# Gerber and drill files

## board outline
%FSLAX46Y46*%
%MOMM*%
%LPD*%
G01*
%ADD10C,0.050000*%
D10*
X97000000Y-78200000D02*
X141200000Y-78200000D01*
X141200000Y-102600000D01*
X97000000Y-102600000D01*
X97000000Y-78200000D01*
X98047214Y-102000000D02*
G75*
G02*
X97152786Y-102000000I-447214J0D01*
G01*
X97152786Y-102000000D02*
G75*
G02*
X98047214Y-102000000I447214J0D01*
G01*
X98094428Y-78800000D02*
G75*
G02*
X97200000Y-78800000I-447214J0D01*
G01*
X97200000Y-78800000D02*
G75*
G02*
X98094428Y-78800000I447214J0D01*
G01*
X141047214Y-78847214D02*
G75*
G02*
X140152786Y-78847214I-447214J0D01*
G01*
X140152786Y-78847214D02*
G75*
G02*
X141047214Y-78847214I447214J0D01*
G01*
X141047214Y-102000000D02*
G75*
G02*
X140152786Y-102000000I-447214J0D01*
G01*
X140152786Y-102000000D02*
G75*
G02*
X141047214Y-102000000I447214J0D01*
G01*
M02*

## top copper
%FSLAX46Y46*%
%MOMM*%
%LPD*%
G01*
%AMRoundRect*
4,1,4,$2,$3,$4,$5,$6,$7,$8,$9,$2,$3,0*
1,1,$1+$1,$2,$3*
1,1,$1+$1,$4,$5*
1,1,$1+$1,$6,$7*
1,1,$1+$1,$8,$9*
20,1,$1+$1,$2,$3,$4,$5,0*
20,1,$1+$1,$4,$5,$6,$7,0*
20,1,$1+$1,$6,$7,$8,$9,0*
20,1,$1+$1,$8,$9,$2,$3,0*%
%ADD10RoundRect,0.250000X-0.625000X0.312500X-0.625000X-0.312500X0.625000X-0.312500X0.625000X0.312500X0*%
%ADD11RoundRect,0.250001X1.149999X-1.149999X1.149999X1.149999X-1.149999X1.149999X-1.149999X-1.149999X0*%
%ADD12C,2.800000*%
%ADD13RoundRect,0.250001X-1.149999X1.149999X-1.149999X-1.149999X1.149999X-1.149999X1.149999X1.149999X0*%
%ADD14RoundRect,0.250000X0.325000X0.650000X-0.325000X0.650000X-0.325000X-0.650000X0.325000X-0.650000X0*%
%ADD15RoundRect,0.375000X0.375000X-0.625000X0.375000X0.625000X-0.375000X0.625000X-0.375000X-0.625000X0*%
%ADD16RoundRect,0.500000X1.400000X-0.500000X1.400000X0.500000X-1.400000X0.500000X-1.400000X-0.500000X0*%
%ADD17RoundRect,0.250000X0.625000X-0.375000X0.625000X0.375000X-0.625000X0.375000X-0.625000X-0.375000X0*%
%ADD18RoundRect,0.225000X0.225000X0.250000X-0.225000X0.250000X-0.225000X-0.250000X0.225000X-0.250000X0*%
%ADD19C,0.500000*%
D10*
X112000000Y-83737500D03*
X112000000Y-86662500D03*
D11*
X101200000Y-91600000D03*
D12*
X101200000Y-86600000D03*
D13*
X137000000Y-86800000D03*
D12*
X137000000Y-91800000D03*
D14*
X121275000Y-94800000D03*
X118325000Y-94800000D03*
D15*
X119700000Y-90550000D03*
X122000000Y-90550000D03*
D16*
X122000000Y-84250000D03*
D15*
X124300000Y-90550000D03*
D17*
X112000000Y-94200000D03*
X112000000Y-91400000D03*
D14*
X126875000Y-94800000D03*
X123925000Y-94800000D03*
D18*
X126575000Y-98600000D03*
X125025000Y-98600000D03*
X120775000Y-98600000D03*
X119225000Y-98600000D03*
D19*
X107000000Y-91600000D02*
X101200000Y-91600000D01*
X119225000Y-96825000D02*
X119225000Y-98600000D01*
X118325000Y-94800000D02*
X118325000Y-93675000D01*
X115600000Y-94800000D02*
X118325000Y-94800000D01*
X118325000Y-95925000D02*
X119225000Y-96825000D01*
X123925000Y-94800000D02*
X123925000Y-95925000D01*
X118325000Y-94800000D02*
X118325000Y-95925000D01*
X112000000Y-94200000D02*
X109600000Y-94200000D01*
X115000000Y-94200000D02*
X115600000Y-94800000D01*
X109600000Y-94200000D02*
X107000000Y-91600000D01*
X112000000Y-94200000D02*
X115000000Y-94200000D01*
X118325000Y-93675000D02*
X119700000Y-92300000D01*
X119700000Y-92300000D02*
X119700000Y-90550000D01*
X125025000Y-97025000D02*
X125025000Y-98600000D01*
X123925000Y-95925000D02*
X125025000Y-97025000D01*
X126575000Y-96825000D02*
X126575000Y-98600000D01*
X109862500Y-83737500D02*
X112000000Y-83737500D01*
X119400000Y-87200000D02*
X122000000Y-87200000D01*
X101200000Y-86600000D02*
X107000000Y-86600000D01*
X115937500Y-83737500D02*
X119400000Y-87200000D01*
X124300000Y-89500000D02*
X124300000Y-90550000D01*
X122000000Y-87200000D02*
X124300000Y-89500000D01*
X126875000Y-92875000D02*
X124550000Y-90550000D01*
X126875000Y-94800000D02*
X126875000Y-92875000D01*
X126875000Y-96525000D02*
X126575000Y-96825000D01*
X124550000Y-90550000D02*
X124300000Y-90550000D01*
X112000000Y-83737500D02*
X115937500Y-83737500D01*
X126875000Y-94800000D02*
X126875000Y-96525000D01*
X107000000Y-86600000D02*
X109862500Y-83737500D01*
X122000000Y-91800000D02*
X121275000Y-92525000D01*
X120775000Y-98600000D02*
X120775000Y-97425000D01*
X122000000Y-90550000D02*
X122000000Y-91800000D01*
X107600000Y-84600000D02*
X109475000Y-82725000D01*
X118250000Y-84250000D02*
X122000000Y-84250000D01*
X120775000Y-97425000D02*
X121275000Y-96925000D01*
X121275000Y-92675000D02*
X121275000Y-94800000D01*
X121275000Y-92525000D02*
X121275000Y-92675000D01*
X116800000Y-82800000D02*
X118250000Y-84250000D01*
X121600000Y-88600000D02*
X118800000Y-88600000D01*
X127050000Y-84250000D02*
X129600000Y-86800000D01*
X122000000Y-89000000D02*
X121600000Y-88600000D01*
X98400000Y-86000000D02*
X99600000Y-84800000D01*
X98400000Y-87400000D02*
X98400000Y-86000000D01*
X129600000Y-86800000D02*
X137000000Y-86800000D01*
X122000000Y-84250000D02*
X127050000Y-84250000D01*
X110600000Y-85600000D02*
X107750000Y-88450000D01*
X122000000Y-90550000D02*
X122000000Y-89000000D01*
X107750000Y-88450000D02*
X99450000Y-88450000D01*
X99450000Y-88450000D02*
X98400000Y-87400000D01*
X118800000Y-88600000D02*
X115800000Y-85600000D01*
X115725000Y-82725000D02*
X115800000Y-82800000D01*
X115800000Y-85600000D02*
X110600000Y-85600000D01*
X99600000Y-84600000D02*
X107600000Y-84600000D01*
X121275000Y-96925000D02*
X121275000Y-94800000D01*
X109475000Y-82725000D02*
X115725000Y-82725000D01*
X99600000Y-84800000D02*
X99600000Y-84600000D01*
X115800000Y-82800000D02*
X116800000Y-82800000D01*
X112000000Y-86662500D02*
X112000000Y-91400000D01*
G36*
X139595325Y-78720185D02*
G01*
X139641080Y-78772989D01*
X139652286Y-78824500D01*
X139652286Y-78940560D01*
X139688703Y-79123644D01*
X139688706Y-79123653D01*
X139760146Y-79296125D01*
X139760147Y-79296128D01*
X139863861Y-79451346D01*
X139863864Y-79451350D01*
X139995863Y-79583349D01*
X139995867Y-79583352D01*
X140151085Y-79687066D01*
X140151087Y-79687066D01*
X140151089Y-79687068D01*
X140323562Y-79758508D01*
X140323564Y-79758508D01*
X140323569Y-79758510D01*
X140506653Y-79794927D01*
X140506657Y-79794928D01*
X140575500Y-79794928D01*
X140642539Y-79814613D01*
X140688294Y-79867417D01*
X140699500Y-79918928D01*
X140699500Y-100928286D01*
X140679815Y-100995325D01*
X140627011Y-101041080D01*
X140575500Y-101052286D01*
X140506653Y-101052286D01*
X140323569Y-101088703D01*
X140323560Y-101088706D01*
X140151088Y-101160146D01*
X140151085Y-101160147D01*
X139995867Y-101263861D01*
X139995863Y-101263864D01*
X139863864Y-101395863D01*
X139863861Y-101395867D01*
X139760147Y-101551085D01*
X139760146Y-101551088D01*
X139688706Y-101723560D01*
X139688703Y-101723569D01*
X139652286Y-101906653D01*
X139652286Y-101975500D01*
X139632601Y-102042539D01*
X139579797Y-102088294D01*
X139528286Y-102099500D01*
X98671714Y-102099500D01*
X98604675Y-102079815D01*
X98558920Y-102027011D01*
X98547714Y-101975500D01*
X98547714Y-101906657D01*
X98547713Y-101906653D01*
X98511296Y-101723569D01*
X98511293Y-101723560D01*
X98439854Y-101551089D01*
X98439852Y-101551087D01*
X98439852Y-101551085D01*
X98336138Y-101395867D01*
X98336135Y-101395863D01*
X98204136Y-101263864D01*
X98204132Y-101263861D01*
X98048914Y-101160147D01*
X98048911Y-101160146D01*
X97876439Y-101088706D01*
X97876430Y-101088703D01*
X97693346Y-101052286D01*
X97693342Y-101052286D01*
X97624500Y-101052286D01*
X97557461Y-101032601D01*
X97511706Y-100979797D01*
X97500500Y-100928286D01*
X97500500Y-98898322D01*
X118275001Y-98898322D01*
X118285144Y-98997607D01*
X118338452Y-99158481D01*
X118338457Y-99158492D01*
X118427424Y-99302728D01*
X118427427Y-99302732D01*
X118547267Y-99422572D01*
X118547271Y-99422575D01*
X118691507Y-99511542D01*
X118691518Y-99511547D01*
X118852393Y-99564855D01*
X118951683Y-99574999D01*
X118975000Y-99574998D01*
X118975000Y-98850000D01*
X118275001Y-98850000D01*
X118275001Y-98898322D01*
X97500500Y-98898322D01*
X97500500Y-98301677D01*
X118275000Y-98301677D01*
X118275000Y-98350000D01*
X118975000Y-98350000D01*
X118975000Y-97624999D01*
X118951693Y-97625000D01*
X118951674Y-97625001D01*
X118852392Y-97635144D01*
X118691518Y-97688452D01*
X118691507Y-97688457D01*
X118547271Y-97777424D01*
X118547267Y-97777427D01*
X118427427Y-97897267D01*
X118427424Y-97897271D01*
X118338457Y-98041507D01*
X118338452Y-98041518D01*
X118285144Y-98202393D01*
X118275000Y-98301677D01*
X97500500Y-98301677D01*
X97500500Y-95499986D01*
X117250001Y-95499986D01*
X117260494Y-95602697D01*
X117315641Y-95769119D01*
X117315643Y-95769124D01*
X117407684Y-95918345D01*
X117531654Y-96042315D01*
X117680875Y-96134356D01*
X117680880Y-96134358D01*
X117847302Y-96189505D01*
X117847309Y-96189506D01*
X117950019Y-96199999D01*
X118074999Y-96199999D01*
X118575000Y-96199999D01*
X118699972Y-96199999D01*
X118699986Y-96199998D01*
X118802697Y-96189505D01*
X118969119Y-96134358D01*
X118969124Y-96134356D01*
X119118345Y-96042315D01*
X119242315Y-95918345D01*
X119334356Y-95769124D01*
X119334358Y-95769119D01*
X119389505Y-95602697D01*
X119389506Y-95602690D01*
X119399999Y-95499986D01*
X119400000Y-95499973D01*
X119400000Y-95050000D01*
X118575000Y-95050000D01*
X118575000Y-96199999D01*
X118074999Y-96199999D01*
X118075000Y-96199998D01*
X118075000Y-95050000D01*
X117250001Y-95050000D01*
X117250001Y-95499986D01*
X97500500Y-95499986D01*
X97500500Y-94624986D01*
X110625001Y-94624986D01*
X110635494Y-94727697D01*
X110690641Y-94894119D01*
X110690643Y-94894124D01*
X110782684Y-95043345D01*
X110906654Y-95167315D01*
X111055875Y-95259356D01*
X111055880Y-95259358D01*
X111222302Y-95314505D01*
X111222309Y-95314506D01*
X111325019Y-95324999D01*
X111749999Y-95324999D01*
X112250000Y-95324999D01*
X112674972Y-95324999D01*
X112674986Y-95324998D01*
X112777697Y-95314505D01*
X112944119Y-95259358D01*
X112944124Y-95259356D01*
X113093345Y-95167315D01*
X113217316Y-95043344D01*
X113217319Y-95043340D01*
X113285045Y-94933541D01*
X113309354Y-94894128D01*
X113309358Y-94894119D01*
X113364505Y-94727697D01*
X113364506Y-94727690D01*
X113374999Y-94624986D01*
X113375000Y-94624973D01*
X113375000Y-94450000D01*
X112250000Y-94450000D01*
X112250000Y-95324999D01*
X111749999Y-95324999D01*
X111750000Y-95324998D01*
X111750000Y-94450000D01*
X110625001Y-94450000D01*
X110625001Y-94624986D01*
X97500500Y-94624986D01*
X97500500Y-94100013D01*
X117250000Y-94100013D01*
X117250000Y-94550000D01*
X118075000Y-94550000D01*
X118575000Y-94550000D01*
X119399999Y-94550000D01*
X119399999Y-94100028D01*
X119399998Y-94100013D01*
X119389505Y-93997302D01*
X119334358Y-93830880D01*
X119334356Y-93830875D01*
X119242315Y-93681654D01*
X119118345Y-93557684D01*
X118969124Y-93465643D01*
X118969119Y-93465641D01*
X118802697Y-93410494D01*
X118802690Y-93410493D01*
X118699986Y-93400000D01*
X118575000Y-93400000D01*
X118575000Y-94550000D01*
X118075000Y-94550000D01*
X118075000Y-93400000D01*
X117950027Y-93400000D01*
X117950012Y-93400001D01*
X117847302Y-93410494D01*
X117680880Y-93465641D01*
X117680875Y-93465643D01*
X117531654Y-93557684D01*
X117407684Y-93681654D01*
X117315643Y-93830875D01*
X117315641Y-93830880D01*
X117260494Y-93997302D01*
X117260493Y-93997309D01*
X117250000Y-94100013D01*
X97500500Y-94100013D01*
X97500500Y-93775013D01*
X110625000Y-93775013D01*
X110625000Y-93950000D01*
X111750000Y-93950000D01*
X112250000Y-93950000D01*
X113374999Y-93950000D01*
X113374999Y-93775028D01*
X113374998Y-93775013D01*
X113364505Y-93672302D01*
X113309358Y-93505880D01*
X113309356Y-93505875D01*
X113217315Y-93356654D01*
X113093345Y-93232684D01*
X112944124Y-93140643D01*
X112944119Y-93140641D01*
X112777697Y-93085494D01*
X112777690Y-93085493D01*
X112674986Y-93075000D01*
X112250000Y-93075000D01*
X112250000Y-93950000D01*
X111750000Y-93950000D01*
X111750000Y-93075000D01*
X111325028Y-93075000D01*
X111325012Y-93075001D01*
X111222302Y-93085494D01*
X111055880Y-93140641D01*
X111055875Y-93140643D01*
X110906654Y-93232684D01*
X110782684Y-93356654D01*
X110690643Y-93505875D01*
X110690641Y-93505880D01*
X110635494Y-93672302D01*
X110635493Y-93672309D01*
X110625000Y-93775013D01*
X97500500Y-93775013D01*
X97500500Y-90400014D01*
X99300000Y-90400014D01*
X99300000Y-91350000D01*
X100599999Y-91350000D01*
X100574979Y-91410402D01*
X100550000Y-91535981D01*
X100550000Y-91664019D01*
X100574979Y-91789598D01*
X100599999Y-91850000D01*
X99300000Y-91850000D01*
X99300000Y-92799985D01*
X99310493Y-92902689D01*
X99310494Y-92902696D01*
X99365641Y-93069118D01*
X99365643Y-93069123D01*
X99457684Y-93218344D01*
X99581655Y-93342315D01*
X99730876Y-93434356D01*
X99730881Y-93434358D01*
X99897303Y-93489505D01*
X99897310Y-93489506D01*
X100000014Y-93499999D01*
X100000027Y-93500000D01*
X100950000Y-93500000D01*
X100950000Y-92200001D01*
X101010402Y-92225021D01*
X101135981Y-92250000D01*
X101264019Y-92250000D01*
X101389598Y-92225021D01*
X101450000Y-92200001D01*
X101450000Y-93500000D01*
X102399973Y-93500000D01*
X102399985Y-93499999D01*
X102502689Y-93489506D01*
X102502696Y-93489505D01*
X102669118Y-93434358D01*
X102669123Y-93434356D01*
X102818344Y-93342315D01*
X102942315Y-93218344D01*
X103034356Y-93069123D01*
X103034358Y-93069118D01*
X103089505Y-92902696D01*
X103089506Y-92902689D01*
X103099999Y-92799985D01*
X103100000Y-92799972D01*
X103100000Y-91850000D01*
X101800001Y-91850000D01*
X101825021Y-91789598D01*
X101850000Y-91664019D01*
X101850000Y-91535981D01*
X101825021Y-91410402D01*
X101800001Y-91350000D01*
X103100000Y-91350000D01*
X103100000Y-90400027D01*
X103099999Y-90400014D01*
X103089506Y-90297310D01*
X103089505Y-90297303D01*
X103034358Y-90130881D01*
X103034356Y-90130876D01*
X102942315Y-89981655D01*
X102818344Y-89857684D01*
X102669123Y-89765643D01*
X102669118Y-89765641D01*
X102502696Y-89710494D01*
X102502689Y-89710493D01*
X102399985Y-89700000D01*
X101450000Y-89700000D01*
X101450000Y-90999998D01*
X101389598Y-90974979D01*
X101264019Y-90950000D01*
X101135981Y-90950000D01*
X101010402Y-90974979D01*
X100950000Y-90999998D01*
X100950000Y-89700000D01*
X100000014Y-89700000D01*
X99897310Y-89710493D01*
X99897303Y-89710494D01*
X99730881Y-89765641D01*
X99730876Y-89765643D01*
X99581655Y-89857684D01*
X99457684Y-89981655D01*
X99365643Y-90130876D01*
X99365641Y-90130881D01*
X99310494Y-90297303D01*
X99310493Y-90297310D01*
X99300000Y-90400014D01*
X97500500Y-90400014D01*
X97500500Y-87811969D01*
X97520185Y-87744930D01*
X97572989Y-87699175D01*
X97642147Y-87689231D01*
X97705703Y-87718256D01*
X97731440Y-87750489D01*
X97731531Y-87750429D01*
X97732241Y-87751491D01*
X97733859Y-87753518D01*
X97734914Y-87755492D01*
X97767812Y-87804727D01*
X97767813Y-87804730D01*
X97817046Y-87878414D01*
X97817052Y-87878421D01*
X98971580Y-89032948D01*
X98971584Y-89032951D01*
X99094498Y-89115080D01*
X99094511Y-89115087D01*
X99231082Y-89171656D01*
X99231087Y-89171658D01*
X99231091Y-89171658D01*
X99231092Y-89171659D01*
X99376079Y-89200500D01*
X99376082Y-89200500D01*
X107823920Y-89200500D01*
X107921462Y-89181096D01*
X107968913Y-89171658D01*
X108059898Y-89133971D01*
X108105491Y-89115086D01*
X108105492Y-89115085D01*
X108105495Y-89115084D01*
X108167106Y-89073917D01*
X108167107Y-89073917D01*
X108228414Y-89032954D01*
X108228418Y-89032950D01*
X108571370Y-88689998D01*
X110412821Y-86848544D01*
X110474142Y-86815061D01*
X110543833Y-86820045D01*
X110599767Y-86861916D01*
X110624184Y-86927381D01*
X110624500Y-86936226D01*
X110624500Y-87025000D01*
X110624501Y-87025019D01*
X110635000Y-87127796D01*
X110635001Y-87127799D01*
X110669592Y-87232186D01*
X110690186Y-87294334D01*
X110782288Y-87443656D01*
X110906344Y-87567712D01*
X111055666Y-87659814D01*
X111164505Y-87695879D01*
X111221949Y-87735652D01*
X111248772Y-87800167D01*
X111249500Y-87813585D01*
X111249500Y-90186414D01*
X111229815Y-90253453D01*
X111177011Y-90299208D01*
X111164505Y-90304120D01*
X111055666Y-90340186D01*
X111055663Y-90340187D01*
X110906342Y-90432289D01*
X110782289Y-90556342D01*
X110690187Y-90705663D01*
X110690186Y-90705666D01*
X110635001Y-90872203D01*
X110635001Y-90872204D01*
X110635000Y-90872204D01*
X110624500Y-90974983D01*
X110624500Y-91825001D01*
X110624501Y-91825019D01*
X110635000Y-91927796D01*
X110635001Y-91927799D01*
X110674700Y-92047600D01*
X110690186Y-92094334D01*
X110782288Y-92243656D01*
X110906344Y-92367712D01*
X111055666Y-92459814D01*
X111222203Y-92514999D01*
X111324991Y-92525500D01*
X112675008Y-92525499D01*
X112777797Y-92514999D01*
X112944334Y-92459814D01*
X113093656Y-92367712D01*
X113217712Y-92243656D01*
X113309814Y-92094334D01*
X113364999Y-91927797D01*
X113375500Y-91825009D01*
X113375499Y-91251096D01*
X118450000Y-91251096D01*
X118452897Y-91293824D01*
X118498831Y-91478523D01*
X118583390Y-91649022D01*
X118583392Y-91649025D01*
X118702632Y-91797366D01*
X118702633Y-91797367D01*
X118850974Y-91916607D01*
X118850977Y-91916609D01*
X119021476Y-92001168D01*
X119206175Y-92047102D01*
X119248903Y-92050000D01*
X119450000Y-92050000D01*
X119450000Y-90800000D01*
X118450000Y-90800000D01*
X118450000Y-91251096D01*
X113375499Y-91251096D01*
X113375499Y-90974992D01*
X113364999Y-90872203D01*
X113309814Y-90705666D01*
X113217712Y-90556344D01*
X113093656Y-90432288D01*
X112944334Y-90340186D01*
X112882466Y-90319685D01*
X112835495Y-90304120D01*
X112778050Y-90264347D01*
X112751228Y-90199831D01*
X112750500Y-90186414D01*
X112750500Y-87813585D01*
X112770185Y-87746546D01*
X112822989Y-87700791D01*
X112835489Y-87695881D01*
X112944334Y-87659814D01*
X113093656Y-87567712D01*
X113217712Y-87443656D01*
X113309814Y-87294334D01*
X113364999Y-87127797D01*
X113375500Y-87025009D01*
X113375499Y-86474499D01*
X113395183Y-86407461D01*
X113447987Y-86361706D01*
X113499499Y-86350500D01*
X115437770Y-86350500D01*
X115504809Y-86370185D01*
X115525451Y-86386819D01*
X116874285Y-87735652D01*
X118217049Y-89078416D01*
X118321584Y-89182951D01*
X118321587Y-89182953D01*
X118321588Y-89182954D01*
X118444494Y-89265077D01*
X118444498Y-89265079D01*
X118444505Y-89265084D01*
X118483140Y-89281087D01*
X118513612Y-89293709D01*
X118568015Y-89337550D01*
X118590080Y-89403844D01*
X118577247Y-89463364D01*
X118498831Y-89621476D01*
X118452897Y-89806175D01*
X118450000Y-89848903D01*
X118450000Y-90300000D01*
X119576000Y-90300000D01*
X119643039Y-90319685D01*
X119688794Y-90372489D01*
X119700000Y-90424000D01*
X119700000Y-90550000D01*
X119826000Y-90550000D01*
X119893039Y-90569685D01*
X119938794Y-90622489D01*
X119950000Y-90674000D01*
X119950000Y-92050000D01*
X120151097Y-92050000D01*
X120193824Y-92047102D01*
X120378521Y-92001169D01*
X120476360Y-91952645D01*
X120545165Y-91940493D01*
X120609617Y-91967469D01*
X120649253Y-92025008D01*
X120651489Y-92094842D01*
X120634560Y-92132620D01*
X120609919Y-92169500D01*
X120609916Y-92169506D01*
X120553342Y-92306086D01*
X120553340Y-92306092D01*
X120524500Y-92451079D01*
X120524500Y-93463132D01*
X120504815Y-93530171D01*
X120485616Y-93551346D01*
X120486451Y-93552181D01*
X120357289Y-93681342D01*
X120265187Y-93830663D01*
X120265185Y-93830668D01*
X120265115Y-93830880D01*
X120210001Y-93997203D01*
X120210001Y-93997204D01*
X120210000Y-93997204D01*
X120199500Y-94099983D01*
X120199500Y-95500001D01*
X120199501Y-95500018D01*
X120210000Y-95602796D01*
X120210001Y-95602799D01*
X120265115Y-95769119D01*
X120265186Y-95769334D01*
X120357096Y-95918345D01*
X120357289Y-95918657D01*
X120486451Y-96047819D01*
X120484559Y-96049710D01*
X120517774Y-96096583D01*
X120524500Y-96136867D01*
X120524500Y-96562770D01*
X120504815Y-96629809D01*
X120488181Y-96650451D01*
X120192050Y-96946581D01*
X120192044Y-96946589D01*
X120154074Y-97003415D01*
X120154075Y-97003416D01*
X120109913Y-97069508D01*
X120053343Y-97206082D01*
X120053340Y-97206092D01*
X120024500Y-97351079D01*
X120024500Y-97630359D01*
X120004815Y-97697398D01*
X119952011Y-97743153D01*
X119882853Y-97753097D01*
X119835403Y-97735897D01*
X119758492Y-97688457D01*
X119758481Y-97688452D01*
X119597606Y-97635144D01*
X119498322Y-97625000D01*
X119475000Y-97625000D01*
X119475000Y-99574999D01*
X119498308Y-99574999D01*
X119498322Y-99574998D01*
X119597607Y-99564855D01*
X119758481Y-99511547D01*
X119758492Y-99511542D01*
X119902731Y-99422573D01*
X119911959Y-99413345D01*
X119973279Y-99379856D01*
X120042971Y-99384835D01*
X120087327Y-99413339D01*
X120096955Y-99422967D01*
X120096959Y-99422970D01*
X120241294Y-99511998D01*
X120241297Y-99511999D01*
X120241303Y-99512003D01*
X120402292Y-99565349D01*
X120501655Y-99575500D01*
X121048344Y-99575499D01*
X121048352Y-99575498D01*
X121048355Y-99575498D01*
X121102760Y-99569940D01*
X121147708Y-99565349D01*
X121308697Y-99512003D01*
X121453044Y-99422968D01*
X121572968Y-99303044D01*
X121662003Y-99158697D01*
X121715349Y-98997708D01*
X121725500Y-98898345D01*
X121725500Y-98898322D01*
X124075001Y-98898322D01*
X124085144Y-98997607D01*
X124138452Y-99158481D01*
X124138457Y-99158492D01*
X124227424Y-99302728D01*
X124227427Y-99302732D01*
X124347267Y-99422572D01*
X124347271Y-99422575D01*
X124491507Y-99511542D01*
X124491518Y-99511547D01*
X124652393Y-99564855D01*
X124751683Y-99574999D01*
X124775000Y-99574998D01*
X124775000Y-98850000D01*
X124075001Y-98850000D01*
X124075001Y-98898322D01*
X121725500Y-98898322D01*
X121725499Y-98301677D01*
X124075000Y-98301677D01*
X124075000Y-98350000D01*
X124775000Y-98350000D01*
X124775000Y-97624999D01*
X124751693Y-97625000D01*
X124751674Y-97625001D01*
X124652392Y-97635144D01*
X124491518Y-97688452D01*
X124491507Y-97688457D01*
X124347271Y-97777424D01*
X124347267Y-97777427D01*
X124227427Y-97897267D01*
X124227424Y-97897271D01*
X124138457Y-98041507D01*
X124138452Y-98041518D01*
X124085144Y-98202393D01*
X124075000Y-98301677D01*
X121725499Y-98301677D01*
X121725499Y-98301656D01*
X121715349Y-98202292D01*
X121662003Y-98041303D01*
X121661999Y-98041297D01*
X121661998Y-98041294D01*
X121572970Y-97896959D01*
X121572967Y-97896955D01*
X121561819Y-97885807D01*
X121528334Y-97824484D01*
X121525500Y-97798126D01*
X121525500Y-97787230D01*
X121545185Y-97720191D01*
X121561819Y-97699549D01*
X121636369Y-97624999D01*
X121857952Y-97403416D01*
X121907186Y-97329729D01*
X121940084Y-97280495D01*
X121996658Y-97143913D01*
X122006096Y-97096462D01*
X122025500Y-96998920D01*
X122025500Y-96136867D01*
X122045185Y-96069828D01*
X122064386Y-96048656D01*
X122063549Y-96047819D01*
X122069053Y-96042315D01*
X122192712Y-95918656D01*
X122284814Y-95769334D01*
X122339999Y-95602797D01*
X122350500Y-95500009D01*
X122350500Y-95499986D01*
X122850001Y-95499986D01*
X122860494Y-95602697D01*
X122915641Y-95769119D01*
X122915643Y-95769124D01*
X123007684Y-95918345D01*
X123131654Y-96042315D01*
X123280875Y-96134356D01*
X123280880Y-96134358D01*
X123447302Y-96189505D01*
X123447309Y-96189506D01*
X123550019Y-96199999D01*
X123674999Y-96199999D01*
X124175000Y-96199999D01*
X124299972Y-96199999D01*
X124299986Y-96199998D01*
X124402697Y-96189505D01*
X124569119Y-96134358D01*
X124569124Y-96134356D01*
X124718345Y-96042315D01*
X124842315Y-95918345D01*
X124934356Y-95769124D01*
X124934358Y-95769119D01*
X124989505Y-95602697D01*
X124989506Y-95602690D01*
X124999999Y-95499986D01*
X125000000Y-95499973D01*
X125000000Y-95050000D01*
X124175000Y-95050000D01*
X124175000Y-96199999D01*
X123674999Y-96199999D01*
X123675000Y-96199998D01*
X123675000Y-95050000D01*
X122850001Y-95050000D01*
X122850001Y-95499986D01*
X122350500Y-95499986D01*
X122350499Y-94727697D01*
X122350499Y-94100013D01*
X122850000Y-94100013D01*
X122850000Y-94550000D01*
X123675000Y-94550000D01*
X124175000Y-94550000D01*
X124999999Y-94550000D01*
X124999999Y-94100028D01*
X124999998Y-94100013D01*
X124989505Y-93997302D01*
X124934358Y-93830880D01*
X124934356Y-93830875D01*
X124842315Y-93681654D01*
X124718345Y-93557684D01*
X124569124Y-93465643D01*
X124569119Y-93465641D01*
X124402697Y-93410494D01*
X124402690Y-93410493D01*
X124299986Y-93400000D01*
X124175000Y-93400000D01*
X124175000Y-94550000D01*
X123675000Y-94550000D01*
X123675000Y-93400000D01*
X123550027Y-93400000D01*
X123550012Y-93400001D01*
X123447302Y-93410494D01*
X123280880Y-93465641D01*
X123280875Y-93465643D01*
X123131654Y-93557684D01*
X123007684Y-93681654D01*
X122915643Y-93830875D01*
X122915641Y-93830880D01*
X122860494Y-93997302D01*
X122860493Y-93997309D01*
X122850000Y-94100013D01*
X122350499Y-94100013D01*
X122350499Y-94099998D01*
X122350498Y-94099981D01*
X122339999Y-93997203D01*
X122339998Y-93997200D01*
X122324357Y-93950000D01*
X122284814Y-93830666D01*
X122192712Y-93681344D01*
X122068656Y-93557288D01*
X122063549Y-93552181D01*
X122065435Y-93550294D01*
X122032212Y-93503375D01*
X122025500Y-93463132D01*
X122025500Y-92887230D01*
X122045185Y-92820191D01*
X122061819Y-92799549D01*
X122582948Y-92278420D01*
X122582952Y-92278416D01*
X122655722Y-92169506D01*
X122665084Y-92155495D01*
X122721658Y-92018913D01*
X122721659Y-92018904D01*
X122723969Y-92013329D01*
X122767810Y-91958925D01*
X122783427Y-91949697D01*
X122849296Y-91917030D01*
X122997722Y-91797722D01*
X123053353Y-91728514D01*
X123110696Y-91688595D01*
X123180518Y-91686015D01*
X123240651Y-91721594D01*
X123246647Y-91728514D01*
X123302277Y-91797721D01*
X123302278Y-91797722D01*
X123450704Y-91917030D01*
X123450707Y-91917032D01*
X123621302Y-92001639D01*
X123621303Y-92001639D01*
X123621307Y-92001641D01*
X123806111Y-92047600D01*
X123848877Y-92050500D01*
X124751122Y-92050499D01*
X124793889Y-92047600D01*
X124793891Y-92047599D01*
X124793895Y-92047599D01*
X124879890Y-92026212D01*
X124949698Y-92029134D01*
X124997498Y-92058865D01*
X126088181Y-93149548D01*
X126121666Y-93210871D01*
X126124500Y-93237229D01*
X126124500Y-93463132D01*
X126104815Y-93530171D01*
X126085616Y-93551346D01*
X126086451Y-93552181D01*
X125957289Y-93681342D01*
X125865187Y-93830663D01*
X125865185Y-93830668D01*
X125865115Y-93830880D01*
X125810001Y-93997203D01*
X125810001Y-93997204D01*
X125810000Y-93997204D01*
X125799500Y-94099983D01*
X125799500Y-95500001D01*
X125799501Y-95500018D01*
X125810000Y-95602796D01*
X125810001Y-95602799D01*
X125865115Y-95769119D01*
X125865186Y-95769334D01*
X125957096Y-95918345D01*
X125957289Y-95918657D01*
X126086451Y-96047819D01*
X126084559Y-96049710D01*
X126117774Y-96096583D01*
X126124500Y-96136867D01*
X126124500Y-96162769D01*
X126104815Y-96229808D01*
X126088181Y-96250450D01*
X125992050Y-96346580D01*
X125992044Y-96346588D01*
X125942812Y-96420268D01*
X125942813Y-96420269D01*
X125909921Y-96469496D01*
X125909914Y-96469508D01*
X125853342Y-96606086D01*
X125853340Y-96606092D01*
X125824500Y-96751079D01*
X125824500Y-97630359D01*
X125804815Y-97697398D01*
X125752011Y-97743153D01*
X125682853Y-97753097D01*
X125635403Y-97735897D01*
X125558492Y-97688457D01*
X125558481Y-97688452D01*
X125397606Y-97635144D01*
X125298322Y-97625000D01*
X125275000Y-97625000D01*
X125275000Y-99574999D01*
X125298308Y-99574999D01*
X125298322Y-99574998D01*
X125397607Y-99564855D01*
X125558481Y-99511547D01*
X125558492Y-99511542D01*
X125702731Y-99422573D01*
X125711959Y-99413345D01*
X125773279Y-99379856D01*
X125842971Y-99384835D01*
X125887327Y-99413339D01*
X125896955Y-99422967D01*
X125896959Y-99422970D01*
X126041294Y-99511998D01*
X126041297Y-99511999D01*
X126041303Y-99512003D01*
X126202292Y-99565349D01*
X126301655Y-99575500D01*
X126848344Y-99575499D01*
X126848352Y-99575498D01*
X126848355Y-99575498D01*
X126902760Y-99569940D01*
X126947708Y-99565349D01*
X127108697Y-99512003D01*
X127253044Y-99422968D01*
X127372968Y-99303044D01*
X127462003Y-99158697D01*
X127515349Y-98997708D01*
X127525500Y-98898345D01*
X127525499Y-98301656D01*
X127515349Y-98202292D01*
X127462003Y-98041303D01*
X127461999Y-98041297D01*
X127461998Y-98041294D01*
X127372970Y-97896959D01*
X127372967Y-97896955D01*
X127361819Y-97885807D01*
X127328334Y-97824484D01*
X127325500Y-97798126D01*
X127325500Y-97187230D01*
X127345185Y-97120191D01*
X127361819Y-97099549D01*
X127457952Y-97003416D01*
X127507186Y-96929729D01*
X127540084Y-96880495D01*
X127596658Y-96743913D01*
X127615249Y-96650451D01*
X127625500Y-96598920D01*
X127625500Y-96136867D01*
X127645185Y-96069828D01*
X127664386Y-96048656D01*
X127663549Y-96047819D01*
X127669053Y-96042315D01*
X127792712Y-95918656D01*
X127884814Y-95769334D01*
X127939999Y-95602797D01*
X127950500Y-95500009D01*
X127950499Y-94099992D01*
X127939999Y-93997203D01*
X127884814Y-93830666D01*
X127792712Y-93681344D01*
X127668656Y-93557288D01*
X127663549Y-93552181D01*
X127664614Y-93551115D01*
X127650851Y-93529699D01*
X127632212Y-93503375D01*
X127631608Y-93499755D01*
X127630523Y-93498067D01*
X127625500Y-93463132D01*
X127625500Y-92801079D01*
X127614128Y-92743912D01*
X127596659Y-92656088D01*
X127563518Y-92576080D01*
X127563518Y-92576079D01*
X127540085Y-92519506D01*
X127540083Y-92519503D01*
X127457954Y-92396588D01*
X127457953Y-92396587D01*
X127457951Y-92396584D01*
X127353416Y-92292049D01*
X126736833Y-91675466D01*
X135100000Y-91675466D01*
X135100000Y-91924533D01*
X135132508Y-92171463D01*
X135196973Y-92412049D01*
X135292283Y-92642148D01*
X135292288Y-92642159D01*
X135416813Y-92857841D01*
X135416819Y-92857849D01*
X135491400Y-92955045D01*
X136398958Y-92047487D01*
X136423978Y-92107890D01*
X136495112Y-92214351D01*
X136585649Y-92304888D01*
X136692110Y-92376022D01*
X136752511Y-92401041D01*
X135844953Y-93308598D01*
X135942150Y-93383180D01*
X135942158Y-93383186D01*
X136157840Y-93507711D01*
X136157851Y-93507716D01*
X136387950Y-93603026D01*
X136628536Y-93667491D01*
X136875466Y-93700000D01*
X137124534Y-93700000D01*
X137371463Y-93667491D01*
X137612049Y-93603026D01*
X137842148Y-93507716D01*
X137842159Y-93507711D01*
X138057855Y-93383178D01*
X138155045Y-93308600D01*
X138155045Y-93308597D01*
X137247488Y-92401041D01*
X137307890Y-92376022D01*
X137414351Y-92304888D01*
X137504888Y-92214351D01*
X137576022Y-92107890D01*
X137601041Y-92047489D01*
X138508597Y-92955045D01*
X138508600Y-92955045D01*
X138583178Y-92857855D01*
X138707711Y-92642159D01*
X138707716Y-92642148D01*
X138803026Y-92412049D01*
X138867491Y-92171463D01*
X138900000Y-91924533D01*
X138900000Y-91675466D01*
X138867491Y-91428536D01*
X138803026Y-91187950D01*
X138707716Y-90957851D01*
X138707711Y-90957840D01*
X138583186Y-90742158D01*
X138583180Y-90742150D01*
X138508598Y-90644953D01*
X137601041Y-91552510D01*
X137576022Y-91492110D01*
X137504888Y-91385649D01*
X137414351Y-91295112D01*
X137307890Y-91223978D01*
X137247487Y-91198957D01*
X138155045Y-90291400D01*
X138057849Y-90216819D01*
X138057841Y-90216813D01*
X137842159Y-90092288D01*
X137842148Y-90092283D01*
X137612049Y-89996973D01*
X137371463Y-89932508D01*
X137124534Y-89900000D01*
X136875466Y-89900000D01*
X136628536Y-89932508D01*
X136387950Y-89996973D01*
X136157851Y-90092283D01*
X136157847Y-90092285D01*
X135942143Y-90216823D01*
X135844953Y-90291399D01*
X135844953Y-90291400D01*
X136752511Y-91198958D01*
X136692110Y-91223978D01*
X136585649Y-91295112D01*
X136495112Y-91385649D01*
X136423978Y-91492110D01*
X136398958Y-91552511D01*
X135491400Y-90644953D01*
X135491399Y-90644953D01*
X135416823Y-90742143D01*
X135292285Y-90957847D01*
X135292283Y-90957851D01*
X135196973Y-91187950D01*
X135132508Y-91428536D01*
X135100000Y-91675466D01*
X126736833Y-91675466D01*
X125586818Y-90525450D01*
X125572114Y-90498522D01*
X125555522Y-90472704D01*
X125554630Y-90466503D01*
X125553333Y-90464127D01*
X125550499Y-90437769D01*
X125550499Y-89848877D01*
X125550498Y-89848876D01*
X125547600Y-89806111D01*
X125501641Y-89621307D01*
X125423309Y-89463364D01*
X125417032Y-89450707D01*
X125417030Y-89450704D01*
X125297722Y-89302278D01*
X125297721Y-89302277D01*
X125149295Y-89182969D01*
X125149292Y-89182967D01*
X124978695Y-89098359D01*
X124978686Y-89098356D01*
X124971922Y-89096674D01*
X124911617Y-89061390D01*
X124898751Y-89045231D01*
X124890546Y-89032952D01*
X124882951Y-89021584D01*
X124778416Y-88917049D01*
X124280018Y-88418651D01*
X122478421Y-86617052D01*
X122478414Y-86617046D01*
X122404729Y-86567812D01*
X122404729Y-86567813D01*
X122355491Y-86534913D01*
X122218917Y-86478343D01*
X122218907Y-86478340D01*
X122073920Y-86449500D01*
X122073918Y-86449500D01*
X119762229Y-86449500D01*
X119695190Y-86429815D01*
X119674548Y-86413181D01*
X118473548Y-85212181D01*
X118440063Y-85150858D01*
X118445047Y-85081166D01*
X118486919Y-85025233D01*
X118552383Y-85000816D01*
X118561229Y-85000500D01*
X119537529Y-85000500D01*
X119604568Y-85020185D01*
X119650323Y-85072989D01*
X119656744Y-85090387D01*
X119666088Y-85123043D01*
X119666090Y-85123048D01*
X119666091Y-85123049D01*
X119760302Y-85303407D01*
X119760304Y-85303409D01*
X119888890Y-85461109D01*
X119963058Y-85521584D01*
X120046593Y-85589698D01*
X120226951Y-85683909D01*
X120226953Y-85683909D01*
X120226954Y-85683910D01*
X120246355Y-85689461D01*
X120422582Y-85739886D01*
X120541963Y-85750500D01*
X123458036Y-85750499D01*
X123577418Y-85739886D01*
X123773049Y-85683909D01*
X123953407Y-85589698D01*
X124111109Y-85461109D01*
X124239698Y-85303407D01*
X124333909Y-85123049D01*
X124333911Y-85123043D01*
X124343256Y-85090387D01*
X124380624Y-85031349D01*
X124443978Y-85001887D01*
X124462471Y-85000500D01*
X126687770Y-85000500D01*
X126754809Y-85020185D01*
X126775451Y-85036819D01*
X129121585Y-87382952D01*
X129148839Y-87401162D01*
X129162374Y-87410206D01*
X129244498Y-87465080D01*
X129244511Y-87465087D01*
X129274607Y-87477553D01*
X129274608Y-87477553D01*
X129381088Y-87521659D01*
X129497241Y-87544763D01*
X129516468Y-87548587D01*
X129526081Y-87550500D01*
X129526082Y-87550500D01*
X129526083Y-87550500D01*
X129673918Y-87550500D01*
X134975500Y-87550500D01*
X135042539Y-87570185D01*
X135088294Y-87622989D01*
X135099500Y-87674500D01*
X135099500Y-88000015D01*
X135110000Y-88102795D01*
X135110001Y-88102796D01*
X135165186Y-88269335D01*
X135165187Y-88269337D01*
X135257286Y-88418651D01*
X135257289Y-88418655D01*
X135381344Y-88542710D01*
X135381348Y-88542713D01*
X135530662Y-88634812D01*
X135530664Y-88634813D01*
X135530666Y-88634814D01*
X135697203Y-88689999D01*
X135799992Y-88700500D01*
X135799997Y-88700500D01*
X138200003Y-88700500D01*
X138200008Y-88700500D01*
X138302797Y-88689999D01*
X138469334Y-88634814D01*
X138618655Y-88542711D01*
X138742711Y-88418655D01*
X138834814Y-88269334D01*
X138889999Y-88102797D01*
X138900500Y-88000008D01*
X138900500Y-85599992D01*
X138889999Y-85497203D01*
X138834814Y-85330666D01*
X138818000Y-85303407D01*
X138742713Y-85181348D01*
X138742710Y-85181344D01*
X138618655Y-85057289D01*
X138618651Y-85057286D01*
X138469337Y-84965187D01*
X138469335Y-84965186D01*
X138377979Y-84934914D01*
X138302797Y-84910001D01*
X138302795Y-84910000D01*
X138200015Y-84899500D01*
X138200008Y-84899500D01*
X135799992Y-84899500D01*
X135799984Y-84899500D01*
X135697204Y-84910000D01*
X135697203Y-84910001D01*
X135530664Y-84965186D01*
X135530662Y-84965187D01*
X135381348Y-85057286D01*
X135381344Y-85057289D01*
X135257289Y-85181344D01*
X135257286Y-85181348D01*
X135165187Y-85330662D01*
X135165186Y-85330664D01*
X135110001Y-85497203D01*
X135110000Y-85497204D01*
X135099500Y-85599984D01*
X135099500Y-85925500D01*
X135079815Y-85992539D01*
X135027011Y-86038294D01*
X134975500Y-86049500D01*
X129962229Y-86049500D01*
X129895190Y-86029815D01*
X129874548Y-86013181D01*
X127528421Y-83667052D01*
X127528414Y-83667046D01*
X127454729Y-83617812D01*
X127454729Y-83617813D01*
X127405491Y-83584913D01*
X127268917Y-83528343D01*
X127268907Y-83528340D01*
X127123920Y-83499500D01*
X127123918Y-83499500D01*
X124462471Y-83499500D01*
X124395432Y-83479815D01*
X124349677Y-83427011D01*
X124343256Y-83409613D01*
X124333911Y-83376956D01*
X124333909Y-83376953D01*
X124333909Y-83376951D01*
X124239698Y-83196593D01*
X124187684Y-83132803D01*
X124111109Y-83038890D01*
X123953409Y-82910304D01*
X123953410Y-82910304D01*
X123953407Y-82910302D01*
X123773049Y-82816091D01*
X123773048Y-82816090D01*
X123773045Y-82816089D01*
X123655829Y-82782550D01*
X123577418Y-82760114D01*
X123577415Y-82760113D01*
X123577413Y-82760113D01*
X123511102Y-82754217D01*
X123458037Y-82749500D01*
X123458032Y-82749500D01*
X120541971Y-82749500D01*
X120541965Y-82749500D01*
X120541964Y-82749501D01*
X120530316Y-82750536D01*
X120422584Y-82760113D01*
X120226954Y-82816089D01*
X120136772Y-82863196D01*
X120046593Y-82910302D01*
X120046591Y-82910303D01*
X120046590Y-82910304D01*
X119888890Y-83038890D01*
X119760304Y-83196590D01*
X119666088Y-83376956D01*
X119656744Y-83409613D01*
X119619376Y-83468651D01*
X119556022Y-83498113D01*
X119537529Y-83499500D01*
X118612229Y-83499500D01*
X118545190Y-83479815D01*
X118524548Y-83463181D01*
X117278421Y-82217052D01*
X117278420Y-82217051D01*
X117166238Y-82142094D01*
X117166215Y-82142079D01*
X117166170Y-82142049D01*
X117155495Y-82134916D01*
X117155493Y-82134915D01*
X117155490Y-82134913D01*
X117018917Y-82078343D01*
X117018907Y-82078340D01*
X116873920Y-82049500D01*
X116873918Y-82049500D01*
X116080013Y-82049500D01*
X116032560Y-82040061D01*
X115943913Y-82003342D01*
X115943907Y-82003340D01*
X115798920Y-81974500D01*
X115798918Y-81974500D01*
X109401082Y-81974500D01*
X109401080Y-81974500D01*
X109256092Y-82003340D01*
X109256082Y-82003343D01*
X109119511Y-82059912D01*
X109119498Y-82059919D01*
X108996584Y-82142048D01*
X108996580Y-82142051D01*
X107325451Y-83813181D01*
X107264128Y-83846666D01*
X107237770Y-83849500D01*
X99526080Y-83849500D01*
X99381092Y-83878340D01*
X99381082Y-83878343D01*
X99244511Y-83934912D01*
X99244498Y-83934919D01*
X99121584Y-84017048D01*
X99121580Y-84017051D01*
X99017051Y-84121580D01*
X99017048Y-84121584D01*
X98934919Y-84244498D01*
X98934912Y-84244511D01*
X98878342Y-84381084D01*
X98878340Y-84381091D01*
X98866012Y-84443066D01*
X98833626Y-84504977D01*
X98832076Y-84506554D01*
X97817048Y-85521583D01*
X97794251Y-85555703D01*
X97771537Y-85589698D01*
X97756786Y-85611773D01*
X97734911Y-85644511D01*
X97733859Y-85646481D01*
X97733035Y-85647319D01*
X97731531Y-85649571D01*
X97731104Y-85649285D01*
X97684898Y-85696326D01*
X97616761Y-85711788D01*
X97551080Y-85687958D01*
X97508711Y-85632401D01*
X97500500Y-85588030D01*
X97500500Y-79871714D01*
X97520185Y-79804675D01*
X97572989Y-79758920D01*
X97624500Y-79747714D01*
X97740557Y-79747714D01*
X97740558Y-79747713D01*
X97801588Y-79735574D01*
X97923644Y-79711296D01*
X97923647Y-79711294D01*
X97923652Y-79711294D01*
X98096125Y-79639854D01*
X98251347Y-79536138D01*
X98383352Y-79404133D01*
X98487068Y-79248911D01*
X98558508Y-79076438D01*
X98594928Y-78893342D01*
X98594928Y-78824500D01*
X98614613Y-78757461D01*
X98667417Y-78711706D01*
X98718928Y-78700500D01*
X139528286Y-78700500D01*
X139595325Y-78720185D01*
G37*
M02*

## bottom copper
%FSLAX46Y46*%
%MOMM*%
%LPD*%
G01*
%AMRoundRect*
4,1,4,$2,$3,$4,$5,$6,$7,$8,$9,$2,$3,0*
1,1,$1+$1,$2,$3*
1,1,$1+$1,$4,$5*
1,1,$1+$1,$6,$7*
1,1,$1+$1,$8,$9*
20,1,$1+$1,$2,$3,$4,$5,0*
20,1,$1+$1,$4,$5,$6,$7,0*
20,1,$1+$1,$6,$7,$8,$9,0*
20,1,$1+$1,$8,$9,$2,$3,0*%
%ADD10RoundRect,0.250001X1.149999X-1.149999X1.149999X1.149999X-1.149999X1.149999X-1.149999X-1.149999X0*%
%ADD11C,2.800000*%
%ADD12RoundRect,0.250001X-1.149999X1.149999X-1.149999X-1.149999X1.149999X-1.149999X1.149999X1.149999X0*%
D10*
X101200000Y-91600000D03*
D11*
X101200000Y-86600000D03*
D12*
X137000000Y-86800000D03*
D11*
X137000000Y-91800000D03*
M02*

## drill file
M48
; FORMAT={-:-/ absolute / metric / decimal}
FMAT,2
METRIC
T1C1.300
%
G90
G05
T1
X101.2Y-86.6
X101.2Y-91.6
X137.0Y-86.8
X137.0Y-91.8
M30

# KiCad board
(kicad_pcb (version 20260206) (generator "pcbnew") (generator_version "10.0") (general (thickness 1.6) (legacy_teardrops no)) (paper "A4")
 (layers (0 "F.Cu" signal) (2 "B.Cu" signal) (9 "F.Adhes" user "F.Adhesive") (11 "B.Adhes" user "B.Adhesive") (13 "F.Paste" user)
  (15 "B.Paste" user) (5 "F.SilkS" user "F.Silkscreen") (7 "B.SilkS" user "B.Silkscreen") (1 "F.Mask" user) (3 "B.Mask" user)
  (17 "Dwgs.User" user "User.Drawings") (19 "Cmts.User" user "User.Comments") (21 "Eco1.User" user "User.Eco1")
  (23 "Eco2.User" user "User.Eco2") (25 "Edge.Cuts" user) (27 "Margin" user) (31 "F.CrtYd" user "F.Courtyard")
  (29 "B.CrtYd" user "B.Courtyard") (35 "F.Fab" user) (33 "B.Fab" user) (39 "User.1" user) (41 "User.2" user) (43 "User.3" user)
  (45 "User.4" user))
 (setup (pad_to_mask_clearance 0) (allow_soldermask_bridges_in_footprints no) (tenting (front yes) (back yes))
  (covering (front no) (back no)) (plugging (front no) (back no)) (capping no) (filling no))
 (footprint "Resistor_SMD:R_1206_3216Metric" (layer "F.Cu") (at 112 85.2 -90)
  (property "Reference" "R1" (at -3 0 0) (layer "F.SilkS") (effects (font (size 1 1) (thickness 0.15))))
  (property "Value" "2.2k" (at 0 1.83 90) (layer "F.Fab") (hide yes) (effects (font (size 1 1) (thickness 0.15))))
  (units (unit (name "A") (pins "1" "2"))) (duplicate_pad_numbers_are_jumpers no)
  (pad "1" smd roundrect (at -1.4625 0 270) (size 1.125 1.75) (layers "F.Cu" "F.Mask" "F.Paste") (roundrect_rratio 0.222222) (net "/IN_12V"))
  (pad "2" smd roundrect (at 1.4625 0 270) (size 1.125 1.75) (layers "F.Cu" "F.Mask" "F.Paste") (roundrect_rratio 0.222222)
   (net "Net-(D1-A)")))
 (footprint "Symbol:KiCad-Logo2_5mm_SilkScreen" (layer "F.Cu") (at 105.156 99.06)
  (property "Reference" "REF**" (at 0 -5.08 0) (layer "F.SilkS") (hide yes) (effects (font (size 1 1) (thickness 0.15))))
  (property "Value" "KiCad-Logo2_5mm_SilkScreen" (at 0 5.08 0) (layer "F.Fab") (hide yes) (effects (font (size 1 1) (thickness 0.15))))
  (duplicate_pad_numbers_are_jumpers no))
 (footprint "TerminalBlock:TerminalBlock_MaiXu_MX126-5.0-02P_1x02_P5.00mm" (layer "F.Cu") (at 101.2 91.6 90)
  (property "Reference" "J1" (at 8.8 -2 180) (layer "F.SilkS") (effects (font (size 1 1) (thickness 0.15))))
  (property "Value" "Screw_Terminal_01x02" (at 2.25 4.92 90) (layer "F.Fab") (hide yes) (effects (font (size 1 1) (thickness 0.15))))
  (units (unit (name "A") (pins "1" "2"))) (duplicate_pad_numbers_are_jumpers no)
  (pad "1" thru_hole roundrect (at 0 0 90) (size 2.8 2.8) (drill 1.3) (layers "*.Cu" "*.Mask") (remove_unused_layers no)
   (roundrect_rratio 0.089286) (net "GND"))
  (pad "2" thru_hole circle (at 5 0 90) (size 2.8 2.8) (drill 1.3) (layers "*.Cu" "*.Mask") (remove_unused_layers no) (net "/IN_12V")))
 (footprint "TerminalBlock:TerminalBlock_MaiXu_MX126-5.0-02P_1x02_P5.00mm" (layer "F.Cu") (at 137 86.8 -90)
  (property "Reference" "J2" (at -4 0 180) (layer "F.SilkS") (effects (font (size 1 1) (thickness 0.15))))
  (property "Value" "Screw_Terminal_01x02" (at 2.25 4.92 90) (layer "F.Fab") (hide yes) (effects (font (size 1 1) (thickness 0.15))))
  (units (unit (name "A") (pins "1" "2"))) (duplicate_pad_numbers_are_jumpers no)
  (pad "1" thru_hole roundrect (at 0 0 270) (size 2.8 2.8) (drill 1.3) (layers "*.Cu" "*.Mask") (remove_unused_layers no)
   (roundrect_rratio 0.089286) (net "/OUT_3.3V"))
  (pad "2" thru_hole circle (at 5 0 270) (size 2.8 2.8) (drill 1.3) (layers "*.Cu" "*.Mask") (remove_unused_layers no) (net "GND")))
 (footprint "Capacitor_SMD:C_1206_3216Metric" (layer "F.Cu") (at 119.8 94.8 180)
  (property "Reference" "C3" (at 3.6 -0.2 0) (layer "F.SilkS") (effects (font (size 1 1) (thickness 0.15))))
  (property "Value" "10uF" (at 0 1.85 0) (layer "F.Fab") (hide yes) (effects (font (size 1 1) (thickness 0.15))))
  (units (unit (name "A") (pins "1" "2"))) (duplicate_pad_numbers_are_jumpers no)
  (pad "1" smd roundrect (at -1.475 0 180) (size 1.15 1.8) (layers "F.Cu" "F.Mask" "F.Paste") (roundrect_rratio 0.217391) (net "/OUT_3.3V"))
  (pad "2" smd roundrect (at 1.475 0 180) (size 1.15 1.8) (layers "F.Cu" "F.Mask" "F.Paste") (roundrect_rratio 0.217391) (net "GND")))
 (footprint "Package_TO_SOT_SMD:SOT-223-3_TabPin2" (layer "F.Cu") (at 122 87.4 90)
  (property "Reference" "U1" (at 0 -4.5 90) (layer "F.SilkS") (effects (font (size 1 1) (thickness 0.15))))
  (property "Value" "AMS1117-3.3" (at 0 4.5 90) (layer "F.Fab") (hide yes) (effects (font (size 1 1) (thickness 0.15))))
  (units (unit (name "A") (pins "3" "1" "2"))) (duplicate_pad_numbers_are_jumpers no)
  (pad "1" smd roundrect (at -3.15 -2.3 90) (size 2 1.5) (layers "F.Cu" "F.Mask" "F.Paste") (roundrect_rratio 0.25) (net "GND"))
  (pad "2" smd roundrect (at -3.15 0 90) (size 2 1.5) (layers "F.Cu" "F.Mask" "F.Paste") (roundrect_rratio 0.25) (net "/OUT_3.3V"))
  (pad "2" smd roundrect (at 3.15 0 90) (size 2 3.8) (layers "F.Cu" "F.Mask" "F.Paste") (roundrect_rratio 0.25) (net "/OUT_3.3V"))
  (pad "3" smd roundrect (at -3.15 2.3 90) (size 2 1.5) (layers "F.Cu" "F.Mask" "F.Paste") (roundrect_rratio 0.25) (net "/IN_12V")))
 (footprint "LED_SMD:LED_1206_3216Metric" (layer "F.Cu") (at 112 92.8 90)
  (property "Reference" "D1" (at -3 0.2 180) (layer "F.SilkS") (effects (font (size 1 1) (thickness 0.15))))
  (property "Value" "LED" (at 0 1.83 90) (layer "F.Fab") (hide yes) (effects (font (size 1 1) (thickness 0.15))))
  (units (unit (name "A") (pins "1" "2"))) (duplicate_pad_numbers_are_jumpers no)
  (pad "1" smd roundrect (at -1.4 0 90) (size 1.25 1.75) (layers "F.Cu" "F.Mask" "F.Paste") (roundrect_rratio 0.2) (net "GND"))
  (pad "2" smd roundrect (at 1.4 0 90) (size 1.25 1.75) (layers "F.Cu" "F.Mask" "F.Paste") (roundrect_rratio 0.2) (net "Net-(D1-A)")))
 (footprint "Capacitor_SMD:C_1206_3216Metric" (layer "F.Cu") (at 125.4 94.8 180)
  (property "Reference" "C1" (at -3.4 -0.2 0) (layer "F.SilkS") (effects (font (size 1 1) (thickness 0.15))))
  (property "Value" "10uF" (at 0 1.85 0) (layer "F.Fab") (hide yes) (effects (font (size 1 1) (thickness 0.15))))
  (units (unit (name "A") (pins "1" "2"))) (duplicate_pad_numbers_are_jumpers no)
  (pad "1" smd roundrect (at -1.475 0 180) (size 1.15 1.8) (layers "F.Cu" "F.Mask" "F.Paste") (roundrect_rratio 0.217391) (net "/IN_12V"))
  (pad "2" smd roundrect (at 1.475 0 180) (size 1.15 1.8) (layers "F.Cu" "F.Mask" "F.Paste") (roundrect_rratio 0.217391) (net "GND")))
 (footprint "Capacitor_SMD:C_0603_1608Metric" (layer "F.Cu") (at 125.8 98.6 180)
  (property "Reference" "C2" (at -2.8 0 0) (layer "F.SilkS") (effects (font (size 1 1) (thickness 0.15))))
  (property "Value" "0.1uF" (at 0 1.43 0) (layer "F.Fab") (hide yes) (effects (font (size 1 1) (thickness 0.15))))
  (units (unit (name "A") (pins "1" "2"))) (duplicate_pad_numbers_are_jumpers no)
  (pad "1" smd roundrect (at -0.775 0 180) (size 0.9 0.95) (layers "F.Cu" "F.Mask" "F.Paste") (roundrect_rratio 0.25) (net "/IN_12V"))
  (pad "2" smd roundrect (at 0.775 0 180) (size 0.9 0.95) (layers "F.Cu" "F.Mask" "F.Paste") (roundrect_rratio 0.25) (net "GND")))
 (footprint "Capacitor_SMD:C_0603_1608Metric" (layer "F.Cu") (at 120 98.6 180)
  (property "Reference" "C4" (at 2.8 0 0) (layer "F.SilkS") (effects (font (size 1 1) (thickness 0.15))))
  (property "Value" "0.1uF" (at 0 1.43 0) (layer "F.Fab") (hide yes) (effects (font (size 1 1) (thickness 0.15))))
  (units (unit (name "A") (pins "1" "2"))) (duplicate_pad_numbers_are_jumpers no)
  (pad "1" smd roundrect (at -0.775 0 180) (size 0.9 0.95) (layers "F.Cu" "F.Mask" "F.Paste") (roundrect_rratio 0.25) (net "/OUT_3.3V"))
  (pad "2" smd roundrect (at 0.775 0 180) (size 0.9 0.95) (layers "F.Cu" "F.Mask" "F.Paste") (roundrect_rratio 0.25) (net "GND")))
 (gr_rect (start 97 78.2) (end 141.2 102.6) (stroke (width 0.05) (type default)) (fill no) (layer "Edge.Cuts"))
 (gr_circle (center 97.6 102) (end 98 102.2) (stroke (width 0.05) (type default)) (fill no) (layer "Edge.Cuts"))
 (gr_circle (center 97.647214 78.8) (end 98.047214 79) (stroke (width 0.05) (type default)) (fill no) (layer "Edge.Cuts"))
 (gr_circle (center 140.6 78.847214) (end 141 79.047214) (stroke (width 0.05) (type default)) (fill no) (layer "Edge.Cuts"))
 (gr_circle (center 140.6 102) (end 141 102.2) (stroke (width 0.05) (type default)) (fill no) (layer "Edge.Cuts"))
 (segment (start 107 91.6) (end 101.2 91.6) (width 0.5) (layer "F.Cu") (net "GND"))
 (segment (start 119.225 96.825) (end 119.225 98.6) (width 0.5) (layer "F.Cu") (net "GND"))
 (segment (start 118.325 94.8) (end 118.325 93.675) (width 0.5) (layer "F.Cu") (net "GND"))
 (segment (start 115.6 94.8) (end 118.325 94.8) (width 0.5) (layer "F.Cu") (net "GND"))
 (segment (start 118.325 95.925) (end 119.225 96.825) (width 0.5) (layer "F.Cu") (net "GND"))
 (segment (start 123.925 94.8) (end 123.925 95.925) (width 0.5) (layer "F.Cu") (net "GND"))
 (segment (start 118.325 94.8) (end 118.325 95.925) (width 0.5) (layer "F.Cu") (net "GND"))
 (segment (start 112 94.2) (end 109.6 94.2) (width 0.5) (layer "F.Cu") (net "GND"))
 (segment (start 115 94.2) (end 115.6 94.8) (width 0.5) (layer "F.Cu") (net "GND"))
 (segment (start 109.6 94.2) (end 107 91.6) (width 0.5) (layer "F.Cu") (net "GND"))
 (segment (start 112 94.2) (end 115 94.2) (width 0.5) (layer "F.Cu") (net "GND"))
 (segment (start 118.325 93.675) (end 119.7 92.3) (width 0.5) (layer "F.Cu") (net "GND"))
 (segment (start 119.7 92.3) (end 119.7 90.55) (width 0.5) (layer "F.Cu") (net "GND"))
 (segment (start 125.025 97.025) (end 125.025 98.6) (width 0.5) (layer "F.Cu") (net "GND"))
 (segment (start 123.925 95.925) (end 125.025 97.025) (width 0.5) (layer "F.Cu") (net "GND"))
 (segment (start 126.575 96.825) (end 126.575 98.6) (width 0.5) (layer "F.Cu") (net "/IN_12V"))
 (segment (start 109.8625 83.7375) (end 112 83.7375) (width 0.5) (layer "F.Cu") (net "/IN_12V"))
 (segment (start 119.4 87.2) (end 122 87.2) (width 0.5) (layer "F.Cu") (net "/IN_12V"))
 (segment (start 101.2 86.6) (end 107 86.6) (width 0.5) (layer "F.Cu") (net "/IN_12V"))
 (segment (start 115.9375 83.7375) (end 119.4 87.2) (width 0.5) (layer "F.Cu") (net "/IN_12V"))
 (segment (start 124.3 89.5) (end 124.3 90.55) (width 0.5) (layer "F.Cu") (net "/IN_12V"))
 (segment (start 122 87.2) (end 124.3 89.5) (width 0.5) (layer "F.Cu") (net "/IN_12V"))
 (segment (start 126.875 92.875) (end 124.55 90.55) (width 0.5) (layer "F.Cu") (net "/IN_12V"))
 (segment (start 126.875 94.8) (end 126.875 92.875) (width 0.5) (layer "F.Cu") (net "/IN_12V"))
 (segment (start 126.875 96.525) (end 126.575 96.825) (width 0.5) (layer "F.Cu") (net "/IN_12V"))
 (segment (start 124.55 90.55) (end 124.3 90.55) (width 0.5) (layer "F.Cu") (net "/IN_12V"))
 (segment (start 112 83.7375) (end 115.9375 83.7375) (width 0.5) (layer "F.Cu") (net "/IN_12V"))
 (segment (start 126.875 94.8) (end 126.875 96.525) (width 0.5) (layer "F.Cu") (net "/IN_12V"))
 (segment (start 107 86.6) (end 109.8625 83.7375) (width 0.5) (layer "F.Cu") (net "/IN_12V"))
 (segment (start 122 91.8) (end 121.275 92.525) (width 0.5) (layer "F.Cu") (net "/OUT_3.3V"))
 (segment (start 120.775 98.6) (end 120.775 97.425) (width 0.5) (layer "F.Cu") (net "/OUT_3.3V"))
 (segment (start 122 90.55) (end 122 91.8) (width 0.5) (layer "F.Cu") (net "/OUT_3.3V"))
 (segment (start 107.6 84.6) (end 109.475 82.725) (width 0.5) (layer "F.Cu") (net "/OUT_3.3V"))
 (segment (start 118.25 84.25) (end 122 84.25) (width 0.5) (layer "F.Cu") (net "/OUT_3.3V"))
 (segment (start 120.775 97.425) (end 121.275 96.925) (width 0.5) (layer "F.Cu") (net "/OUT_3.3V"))
 (segment (start 121.275 92.675) (end 121.275 94.8) (width 0.5) (layer "F.Cu") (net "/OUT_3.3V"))
 (segment (start 121.275 92.525) (end 121.275 92.675) (width 0.5) (layer "F.Cu") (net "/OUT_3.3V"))
 (segment (start 116.8 82.8) (end 118.25 84.25) (width 0.5) (layer "F.Cu") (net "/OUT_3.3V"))
 (segment (start 121.6 88.6) (end 118.8 88.6) (width 0.5) (layer "F.Cu") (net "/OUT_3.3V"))
 (segment (start 127.05 84.25) (end 129.6 86.8) (width 0.5) (layer "F.Cu") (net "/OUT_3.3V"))
 (segment (start 122 89) (end 121.6 88.6) (width 0.5) (layer "F.Cu") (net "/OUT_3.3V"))
 (segment (start 98.4 86) (end 99.6 84.8) (width 0.5) (layer "F.Cu") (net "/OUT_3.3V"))
 (segment (start 98.4 87.4) (end 98.4 86) (width 0.5) (layer "F.Cu") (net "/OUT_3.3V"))
 (segment (start 129.6 86.8) (end 137 86.8) (width 0.5) (layer "F.Cu") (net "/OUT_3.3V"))
 (segment (start 122 84.25) (end 127.05 84.25) (width 0.5) (layer "F.Cu") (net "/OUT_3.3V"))
 (segment (start 110.6 85.6) (end 107.75 88.45) (width 0.5) (layer "F.Cu") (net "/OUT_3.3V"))
 (segment (start 122 90.55) (end 122 89) (width 0.5) (layer "F.Cu") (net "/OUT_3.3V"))
 (segment (start 107.75 88.45) (end 99.45 88.45) (width 0.5) (layer "F.Cu") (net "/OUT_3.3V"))
 (segment (start 99.45 88.45) (end 98.4 87.4) (width 0.5) (layer "F.Cu") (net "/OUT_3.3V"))
 (segment (start 118.8 88.6) (end 115.8 85.6) (width 0.5) (layer "F.Cu") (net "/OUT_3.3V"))
 (segment (start 115.725 82.725) (end 115.8 82.8) (width 0.5) (layer "F.Cu") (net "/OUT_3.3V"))
 (segment (start 115.8 85.6) (end 110.6 85.6) (width 0.5) (layer "F.Cu") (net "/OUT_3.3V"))
 (segment (start 99.6 84.6) (end 107.6 84.6) (width 0.5) (layer "F.Cu") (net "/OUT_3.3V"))
 (segment (start 121.275 96.925) (end 121.275 94.8) (width 0.5) (layer "F.Cu") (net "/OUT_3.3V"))
 (segment (start 109.475 82.725) (end 115.725 82.725) (width 0.5) (layer "F.Cu") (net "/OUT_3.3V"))
 (segment (start 99.6 84.8) (end 99.6 84.6) (width 0.5) (layer "F.Cu") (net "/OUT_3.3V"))
 (segment (start 115.8 82.8) (end 116.8 82.8) (width 0.5) (layer "F.Cu") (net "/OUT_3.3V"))
 (segment (start 112 86.6625) (end 112 91.4) (width 0.5) (layer "F.Cu") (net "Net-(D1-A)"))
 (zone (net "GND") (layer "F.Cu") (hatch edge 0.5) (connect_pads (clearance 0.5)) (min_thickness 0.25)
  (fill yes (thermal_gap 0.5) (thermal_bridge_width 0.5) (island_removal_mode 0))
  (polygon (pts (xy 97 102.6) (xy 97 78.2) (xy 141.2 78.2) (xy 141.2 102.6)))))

